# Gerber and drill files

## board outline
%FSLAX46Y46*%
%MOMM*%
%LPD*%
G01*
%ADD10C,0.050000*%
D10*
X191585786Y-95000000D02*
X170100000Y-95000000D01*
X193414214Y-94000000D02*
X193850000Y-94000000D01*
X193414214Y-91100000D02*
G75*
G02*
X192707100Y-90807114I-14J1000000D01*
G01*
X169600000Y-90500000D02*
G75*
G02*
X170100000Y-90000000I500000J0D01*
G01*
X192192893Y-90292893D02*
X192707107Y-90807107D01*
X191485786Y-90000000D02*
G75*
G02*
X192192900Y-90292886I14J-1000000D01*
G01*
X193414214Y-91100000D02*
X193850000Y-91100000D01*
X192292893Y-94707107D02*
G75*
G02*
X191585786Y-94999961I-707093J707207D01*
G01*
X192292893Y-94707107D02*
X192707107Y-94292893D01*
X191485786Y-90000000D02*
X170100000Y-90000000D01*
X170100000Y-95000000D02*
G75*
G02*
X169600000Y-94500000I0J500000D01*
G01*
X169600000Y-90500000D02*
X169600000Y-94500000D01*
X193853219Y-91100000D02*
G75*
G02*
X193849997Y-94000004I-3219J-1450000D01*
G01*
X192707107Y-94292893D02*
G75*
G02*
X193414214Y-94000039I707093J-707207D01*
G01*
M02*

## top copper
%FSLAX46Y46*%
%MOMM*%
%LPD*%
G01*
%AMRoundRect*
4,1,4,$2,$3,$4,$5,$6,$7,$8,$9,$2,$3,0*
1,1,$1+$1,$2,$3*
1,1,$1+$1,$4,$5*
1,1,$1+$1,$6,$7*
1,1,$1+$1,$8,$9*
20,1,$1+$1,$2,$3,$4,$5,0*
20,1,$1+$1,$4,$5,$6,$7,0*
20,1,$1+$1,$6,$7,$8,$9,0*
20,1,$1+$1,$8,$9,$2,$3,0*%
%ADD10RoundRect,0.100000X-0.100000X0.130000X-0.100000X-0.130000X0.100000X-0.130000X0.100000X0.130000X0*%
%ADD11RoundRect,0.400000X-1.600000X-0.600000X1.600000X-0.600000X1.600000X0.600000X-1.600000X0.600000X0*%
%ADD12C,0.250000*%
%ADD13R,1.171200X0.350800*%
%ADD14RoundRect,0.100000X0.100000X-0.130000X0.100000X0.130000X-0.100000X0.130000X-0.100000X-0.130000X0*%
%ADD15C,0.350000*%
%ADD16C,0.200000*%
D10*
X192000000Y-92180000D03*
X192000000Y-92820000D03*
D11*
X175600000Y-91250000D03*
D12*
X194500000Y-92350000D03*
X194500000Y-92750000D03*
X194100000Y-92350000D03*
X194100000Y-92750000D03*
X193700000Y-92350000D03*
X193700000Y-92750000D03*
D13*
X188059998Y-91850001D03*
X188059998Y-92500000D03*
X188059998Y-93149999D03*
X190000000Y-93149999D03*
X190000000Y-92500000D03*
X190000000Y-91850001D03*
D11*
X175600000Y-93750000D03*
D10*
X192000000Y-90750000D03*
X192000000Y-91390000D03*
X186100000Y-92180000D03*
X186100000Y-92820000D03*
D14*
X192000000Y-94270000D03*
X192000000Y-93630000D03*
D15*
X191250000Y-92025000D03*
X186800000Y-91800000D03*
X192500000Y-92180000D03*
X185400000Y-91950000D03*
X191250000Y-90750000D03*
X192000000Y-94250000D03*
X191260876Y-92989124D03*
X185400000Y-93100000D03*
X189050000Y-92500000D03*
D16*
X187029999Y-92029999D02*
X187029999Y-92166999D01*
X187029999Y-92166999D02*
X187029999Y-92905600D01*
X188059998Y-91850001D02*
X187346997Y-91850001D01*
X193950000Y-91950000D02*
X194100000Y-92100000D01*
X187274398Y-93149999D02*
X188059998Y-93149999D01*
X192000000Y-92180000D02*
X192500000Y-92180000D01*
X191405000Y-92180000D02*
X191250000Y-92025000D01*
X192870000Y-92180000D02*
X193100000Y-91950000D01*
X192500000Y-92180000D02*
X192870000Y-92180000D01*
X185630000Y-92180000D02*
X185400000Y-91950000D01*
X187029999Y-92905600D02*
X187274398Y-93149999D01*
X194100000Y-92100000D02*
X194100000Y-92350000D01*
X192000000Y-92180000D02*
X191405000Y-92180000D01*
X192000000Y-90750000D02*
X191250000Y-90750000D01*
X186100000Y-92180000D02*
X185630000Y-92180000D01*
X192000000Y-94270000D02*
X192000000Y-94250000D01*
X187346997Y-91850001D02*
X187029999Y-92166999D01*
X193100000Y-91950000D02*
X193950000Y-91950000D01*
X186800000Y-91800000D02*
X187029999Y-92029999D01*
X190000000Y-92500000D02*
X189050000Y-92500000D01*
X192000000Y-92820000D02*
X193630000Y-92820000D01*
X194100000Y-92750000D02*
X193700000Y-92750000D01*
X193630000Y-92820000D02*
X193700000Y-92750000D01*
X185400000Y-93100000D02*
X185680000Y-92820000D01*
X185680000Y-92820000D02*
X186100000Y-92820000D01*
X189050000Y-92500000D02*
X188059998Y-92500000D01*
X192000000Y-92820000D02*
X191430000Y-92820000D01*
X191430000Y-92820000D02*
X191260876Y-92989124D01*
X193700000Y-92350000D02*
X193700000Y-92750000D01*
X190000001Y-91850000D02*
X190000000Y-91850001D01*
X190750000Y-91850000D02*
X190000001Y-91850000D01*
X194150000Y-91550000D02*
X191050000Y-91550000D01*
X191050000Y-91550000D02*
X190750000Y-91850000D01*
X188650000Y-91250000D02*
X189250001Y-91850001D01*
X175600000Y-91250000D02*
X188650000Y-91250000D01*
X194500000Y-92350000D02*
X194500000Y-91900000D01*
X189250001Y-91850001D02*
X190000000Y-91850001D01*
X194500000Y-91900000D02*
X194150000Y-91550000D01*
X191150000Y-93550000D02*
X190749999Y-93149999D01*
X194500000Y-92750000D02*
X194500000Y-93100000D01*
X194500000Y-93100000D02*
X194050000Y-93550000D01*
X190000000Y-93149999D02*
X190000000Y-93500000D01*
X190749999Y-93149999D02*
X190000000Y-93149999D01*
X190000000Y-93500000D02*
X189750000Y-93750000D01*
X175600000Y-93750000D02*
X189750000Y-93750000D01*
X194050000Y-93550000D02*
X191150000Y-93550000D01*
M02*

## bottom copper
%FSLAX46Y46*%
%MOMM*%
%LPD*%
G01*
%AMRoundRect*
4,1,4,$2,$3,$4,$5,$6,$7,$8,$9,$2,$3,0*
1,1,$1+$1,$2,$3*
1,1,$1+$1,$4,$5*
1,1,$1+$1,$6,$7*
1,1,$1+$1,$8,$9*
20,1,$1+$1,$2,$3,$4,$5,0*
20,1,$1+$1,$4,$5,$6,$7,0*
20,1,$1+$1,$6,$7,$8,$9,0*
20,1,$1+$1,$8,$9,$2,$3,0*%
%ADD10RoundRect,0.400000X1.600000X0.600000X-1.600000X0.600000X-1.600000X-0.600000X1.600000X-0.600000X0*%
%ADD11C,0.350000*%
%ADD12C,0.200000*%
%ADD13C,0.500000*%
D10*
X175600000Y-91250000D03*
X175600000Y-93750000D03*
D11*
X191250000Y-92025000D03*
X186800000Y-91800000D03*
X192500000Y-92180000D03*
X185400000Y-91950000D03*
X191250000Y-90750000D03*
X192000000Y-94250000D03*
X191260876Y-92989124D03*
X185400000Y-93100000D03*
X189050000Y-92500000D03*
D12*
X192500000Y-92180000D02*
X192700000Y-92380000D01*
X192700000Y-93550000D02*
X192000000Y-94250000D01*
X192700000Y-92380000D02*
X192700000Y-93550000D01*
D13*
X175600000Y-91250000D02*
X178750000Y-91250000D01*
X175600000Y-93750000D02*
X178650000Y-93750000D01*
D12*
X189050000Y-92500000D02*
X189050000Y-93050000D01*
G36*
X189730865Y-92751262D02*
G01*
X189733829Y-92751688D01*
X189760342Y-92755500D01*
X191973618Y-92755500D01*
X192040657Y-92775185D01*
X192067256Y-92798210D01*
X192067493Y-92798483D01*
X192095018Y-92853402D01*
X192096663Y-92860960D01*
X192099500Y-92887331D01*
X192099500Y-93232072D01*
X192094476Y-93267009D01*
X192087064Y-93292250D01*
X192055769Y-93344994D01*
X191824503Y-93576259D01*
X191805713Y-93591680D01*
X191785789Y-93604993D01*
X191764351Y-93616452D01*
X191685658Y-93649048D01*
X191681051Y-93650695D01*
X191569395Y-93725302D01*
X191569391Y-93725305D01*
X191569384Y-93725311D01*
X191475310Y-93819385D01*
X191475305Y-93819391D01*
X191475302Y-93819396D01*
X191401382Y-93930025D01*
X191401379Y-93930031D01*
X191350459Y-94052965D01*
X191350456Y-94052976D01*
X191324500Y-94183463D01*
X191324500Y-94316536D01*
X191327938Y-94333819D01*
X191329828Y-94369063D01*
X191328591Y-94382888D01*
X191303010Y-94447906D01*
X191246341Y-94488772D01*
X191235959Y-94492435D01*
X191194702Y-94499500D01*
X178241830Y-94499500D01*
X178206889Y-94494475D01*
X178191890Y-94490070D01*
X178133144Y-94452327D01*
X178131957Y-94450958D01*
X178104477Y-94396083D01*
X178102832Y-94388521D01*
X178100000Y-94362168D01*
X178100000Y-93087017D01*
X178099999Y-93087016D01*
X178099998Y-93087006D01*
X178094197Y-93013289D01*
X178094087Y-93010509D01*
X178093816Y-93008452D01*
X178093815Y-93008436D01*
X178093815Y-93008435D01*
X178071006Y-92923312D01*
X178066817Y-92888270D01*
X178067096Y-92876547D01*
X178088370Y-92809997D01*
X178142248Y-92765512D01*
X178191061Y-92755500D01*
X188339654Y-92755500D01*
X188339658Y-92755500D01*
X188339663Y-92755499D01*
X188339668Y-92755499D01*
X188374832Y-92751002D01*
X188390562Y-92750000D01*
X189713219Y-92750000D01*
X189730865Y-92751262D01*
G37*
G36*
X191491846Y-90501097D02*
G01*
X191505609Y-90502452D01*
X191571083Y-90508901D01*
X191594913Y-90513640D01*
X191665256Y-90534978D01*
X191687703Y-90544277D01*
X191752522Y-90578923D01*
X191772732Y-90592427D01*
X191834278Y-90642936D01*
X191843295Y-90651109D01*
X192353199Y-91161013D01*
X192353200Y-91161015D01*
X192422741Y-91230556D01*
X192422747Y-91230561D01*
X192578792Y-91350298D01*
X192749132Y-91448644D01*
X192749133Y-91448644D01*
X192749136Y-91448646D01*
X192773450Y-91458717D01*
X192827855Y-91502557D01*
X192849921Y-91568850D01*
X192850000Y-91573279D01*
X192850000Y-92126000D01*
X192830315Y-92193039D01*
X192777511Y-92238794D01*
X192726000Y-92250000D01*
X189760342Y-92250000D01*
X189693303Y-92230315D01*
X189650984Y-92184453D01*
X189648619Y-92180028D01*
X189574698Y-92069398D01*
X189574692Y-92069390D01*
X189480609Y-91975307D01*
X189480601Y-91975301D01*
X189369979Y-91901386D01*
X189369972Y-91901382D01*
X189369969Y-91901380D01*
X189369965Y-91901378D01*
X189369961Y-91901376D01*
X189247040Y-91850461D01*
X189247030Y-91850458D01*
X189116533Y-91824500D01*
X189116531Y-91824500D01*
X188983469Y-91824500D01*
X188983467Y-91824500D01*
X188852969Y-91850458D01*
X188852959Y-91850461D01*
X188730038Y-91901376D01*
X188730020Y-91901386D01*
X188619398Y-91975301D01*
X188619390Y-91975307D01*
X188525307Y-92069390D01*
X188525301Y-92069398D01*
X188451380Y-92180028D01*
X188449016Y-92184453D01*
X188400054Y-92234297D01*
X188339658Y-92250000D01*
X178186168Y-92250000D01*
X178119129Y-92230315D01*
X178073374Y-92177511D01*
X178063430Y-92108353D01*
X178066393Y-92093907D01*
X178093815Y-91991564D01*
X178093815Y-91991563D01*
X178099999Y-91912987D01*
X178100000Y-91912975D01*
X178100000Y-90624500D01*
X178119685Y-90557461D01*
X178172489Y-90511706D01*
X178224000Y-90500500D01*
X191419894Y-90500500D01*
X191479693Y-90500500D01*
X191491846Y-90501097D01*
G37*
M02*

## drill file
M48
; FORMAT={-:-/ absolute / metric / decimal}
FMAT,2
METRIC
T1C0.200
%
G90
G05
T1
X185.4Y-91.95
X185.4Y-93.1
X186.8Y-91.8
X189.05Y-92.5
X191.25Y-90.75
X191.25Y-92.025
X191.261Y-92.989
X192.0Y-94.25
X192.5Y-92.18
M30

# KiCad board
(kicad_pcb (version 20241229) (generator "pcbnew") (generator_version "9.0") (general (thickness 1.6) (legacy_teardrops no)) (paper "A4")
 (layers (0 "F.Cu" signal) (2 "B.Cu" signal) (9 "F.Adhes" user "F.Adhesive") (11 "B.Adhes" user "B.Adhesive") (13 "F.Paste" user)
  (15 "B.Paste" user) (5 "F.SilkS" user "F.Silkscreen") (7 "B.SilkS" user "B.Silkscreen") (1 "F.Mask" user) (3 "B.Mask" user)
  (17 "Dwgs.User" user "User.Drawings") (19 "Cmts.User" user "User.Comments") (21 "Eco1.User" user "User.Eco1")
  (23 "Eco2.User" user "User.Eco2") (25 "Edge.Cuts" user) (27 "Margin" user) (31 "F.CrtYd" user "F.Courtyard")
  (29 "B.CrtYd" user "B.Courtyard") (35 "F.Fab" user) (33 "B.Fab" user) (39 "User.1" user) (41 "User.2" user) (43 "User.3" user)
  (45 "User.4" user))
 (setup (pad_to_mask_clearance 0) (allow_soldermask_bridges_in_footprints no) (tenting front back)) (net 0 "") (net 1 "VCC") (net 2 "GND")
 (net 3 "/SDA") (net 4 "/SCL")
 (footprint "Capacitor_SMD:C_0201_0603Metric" (layer "F.Cu") (at 192 92.5 -90)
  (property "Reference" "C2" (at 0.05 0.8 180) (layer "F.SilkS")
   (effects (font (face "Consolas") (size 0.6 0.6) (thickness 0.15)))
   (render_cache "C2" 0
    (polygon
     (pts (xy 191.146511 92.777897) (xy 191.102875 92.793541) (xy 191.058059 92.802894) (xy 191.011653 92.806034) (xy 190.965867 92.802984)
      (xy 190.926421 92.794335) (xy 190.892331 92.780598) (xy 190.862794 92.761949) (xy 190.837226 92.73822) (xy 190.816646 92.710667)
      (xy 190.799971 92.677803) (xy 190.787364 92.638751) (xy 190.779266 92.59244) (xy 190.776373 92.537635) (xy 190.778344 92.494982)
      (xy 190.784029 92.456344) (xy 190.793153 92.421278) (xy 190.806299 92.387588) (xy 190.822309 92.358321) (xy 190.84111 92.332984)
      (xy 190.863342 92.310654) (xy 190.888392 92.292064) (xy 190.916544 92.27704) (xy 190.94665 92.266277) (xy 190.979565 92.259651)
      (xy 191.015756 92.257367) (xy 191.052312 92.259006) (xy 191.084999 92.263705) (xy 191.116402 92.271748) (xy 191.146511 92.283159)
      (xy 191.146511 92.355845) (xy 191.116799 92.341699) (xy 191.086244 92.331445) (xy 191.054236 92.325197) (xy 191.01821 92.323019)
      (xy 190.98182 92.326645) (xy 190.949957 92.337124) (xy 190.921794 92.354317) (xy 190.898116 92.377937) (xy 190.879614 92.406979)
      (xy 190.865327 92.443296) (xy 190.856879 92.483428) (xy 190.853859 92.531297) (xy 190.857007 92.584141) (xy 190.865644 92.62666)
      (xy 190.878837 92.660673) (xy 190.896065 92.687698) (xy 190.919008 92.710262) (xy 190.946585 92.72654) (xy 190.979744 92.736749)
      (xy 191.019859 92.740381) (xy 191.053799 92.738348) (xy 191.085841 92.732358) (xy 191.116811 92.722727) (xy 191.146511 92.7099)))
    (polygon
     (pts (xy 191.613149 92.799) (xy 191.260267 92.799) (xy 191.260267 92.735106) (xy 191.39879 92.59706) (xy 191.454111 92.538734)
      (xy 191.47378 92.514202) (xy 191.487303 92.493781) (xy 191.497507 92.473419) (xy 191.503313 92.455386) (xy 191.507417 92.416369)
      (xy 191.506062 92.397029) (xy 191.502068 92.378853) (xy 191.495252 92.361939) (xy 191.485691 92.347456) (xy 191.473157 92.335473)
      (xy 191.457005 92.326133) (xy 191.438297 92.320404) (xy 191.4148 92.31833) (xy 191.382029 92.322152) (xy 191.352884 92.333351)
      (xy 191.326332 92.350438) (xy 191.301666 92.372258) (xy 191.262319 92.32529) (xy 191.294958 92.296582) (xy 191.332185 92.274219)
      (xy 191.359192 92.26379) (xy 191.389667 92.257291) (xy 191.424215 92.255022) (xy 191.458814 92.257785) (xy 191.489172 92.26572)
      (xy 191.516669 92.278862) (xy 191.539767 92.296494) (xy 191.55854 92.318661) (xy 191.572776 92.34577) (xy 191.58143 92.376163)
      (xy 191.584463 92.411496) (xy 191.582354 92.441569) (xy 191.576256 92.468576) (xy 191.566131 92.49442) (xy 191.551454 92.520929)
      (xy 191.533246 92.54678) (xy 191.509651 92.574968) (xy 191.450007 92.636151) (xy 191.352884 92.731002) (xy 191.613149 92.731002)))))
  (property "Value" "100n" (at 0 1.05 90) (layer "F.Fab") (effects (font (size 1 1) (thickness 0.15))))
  (pad "" smd roundrect (at -0.345 0 270) (size 0.318 0.36) (layers "F.Paste") (roundrect_rratio 0.25))
  (pad "" smd roundrect (at 0.345 0 270) (size 0.318 0.36) (layers "F.Paste") (roundrect_rratio 0.25))
  (pad "1" smd roundrect (at -0.32 0 270) (size 0.46 0.4) (layers "F.Cu" "F.Mask") (roundrect_rratio 0.25) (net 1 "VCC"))
  (pad "2" smd roundrect (at 0.32 0 270) (size 0.46 0.4) (layers "F.Cu" "F.Mask") (roundrect_rratio 0.25) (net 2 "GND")))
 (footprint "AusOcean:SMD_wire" (layer "F.Cu") (at 175.6 91.25)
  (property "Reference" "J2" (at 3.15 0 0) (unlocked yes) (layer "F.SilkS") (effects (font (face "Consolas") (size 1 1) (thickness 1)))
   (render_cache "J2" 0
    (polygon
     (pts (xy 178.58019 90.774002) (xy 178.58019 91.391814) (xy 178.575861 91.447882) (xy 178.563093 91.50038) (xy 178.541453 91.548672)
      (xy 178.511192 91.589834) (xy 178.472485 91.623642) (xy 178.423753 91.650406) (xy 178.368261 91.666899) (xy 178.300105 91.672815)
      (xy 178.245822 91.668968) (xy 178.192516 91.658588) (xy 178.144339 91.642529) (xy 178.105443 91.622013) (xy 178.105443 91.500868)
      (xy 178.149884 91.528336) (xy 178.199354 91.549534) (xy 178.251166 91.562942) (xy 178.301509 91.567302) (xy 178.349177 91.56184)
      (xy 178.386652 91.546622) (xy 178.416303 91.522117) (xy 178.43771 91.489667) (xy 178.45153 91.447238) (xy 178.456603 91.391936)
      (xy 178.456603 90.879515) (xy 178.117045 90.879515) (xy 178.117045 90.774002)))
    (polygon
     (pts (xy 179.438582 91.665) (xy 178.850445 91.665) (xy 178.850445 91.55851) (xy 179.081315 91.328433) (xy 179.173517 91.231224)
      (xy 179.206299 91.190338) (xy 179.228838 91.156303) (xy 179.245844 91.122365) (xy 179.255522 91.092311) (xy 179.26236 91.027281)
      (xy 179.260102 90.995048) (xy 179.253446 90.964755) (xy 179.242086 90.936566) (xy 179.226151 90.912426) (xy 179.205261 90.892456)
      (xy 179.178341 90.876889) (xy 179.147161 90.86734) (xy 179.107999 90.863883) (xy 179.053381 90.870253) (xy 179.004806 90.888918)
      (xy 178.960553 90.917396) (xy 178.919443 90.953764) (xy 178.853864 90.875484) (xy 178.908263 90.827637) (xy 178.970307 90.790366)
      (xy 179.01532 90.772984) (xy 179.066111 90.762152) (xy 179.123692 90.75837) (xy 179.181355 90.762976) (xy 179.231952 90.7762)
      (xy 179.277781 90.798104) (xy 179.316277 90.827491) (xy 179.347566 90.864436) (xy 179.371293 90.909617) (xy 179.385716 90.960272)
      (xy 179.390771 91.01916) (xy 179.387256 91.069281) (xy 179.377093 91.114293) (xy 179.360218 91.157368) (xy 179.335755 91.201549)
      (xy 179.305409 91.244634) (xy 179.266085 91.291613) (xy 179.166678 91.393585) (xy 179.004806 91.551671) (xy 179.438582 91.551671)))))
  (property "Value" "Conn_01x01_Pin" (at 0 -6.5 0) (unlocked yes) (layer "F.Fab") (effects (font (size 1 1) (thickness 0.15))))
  (pad "1" smd roundrect (at 0 0) (size 4 2) (layers "F.Cu" "F.Mask" "F.Paste") (roundrect_rratio 0.2) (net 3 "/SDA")
   (thermal_bridge_angle 45)))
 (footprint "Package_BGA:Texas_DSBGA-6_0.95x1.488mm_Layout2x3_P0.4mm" (layer "F.Cu") (at 194.1 92.55 -90)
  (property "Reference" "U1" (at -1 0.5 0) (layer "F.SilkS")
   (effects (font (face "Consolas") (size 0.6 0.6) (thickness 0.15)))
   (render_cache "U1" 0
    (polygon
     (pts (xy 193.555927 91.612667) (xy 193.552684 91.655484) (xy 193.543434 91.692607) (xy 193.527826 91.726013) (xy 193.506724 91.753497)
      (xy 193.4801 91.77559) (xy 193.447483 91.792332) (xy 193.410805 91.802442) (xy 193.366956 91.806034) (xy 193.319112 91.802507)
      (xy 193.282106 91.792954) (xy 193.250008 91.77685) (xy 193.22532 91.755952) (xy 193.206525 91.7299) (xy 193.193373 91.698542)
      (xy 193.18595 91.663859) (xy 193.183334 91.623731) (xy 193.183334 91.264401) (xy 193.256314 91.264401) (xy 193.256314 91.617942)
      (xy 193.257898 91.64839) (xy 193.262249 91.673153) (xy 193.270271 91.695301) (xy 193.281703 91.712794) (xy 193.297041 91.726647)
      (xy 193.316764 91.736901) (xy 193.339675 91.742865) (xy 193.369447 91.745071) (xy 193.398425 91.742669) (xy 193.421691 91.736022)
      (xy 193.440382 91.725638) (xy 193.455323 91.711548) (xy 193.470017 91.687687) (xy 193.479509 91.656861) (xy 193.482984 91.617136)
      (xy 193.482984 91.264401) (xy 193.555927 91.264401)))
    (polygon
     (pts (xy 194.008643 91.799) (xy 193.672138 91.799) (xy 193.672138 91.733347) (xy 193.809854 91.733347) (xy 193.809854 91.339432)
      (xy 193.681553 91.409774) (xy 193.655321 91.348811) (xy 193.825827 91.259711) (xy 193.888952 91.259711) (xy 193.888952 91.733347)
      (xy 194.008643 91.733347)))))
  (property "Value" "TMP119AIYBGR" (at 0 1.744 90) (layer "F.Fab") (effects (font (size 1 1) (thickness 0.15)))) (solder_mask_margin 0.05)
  (pad "A1" smd circle (at -0.2 -0.4 270) (size 0.25 0.25) (layers "F.Cu" "F.Mask" "F.Paste") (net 3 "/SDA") (clearance 0.05))
  (pad "A2" smd circle (at 0.2 -0.4 270) (size 0.25 0.25) (layers "F.Cu" "F.Mask" "F.Paste") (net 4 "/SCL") (clearance 0.05))
  (pad "B1" smd circle (at -0.2 0 270) (size 0.25 0.25) (layers "F.Cu" "F.Mask" "F.Paste") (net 1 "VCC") (clearance 0.05))
  (pad "B2" smd circle (at 0.2 0 270) (size 0.25 0.25) (layers "F.Cu" "F.Mask" "F.Paste") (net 2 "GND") (clearance 0.05))
  (pad "C1" smd circle (at -0.2 0.4 270) (size 0.25 0.25) (layers "F.Cu" "F.Mask" "F.Paste") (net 2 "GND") (clearance 0.05))
  (pad "C2" smd circle (at 0.2 0.4 270) (size 0.25 0.25) (layers "F.Cu" "F.Mask" "F.Paste") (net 2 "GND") (clearance 0.05)))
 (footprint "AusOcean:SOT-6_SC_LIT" (layer "F.Cu") (at 189.029999 92.5)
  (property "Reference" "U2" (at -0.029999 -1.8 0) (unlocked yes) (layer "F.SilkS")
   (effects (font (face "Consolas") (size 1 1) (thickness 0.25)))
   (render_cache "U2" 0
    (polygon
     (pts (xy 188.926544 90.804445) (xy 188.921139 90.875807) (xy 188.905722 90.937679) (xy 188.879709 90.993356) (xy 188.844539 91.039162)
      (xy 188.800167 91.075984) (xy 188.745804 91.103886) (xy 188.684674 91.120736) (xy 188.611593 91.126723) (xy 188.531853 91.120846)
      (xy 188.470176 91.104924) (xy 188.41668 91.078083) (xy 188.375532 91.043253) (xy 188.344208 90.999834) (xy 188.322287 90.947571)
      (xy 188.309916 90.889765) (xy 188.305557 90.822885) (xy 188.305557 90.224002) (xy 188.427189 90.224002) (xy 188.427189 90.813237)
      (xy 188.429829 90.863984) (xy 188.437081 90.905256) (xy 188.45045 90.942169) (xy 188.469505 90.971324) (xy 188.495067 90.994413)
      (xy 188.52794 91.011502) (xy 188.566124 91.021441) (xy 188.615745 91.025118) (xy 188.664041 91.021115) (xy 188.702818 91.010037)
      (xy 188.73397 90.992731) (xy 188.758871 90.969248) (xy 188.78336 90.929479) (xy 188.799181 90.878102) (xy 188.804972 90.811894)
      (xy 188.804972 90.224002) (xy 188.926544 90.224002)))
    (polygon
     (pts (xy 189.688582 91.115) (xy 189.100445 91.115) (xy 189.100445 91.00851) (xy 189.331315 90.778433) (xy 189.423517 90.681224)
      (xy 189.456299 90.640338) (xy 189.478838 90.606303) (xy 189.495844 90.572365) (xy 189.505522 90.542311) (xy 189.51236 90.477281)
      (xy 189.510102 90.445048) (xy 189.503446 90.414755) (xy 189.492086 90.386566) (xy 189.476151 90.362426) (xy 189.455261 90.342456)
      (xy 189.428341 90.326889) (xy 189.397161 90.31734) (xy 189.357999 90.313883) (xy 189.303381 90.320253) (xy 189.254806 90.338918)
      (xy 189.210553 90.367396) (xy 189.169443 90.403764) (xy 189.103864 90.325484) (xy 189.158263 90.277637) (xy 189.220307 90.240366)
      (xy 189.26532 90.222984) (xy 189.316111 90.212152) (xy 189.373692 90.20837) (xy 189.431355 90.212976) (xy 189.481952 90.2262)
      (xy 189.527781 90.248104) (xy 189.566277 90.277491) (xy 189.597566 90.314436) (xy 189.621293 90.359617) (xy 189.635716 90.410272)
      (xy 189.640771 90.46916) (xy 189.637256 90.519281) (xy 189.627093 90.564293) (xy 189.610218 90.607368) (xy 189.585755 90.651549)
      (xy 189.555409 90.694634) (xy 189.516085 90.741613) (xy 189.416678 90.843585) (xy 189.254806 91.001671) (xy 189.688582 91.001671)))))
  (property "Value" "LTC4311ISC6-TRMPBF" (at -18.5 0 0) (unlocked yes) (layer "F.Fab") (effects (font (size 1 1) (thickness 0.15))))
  (pad "1" smd rect (at -0.970001 -0.649999) (size 1.1712 0.3508) (layers "F.Cu" "F.Mask" "F.Paste") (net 1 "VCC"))
  (pad "2" smd rect (at -0.970001 0) (size 1.1712 0.3508) (layers "F.Cu" "F.Mask" "F.Paste") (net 2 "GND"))
  (pad "3" smd rect (at -0.970001 0.649999) (size 1.1712 0.3508) (layers "F.Cu" "F.Mask" "F.Paste") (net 1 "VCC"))
  (pad "4" smd rect (at 0.970001 0.649999) (size 1.1712 0.3508) (layers "F.Cu" "F.Mask" "F.Paste") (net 4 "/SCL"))
  (pad "5" smd rect (at 0.970001 0) (size 1.1712 0.3508) (layers "F.Cu" "F.Mask" "F.Paste") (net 2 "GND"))
  (pad "6" smd rect (at 0.970001 -0.649999) (size 1.1712 0.3508) (layers "F.Cu" "F.Mask" "F.Paste") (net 3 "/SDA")))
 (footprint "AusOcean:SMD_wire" (layer "F.Cu") (at 175.6 93.75)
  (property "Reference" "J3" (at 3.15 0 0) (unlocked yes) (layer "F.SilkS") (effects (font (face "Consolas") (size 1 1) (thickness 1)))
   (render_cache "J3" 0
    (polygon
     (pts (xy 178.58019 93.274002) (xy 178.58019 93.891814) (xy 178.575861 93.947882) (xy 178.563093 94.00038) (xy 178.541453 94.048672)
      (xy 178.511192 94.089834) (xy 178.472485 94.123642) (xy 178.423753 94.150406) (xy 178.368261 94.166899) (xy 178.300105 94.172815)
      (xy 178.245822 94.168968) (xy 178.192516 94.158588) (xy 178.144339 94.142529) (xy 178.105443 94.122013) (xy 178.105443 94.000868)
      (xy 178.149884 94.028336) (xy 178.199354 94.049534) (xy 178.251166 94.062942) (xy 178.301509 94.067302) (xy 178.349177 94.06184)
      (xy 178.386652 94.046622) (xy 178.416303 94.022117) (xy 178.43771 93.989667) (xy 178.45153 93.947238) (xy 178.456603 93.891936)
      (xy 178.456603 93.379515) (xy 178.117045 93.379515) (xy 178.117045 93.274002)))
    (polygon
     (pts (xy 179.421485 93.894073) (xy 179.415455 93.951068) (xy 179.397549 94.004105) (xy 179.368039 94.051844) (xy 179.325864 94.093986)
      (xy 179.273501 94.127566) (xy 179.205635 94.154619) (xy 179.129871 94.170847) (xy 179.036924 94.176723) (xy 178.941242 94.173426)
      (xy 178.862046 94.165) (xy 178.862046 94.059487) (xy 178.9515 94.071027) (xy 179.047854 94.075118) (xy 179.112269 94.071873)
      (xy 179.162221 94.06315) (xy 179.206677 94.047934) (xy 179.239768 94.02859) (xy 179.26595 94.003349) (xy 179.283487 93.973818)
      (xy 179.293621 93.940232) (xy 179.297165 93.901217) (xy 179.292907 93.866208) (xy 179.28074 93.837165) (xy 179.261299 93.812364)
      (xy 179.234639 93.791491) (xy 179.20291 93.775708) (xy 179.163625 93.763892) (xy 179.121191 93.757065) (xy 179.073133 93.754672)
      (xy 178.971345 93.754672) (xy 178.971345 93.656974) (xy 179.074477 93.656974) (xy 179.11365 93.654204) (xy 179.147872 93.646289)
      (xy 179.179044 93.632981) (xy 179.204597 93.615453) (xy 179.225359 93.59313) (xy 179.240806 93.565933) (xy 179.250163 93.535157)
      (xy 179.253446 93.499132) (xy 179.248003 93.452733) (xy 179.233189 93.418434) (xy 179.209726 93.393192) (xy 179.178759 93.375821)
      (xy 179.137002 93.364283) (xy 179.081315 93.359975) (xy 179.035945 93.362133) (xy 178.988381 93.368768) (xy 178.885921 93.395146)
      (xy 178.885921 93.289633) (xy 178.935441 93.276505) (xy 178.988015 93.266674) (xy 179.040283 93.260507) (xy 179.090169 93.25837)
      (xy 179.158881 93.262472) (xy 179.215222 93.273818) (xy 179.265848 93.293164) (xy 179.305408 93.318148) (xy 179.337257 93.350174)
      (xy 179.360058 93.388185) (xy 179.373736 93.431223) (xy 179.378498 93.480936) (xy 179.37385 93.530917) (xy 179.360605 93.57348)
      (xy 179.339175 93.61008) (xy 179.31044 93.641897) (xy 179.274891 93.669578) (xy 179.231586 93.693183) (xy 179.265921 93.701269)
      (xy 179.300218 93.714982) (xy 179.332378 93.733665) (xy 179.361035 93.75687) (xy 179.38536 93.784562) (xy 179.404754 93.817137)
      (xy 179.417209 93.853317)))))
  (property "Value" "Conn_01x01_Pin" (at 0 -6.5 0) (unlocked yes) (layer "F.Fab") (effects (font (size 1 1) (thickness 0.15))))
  (pad "1" smd roundrect (at 0 0) (size 4 2) (layers "F.Cu" "F.Mask" "F.Paste") (roundrect_rratio 0.2) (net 4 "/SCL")
   (thermal_bridge_angle 45)))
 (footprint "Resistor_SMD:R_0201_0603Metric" (layer "F.Cu") (at 192 91.07 -90)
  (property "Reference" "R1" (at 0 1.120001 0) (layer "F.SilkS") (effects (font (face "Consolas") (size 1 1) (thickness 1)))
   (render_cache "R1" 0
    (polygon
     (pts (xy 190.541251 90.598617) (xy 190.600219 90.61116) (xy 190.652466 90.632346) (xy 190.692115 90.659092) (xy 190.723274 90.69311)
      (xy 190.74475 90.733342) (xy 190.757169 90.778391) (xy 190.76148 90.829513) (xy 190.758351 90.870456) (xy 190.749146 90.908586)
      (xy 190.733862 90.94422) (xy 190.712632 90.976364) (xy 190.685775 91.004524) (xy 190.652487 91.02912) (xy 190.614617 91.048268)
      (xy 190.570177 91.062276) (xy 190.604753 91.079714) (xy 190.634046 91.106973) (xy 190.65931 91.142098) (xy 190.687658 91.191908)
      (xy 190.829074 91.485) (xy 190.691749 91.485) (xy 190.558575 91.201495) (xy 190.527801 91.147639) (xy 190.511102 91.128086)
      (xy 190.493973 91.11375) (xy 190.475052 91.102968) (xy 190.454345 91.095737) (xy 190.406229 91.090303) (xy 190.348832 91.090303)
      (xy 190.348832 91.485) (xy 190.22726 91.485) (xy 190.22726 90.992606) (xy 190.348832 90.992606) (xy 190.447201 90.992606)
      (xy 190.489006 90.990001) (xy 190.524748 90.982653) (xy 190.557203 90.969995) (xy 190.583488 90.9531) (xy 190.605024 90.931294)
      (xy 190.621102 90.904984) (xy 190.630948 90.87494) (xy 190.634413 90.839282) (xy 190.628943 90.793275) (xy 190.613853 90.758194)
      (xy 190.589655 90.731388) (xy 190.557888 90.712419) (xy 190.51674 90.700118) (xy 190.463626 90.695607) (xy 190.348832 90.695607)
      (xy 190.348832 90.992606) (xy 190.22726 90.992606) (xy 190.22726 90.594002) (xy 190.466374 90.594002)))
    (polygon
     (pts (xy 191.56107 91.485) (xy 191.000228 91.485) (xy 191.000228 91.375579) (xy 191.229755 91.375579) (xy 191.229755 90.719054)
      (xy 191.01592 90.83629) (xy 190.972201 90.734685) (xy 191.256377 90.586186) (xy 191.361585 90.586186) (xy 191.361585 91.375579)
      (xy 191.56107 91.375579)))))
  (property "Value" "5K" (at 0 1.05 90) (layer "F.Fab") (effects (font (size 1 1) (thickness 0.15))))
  (pad "" smd roundrect (at -0.345 0 270) (size 0.318 0.36) (layers "F.Paste") (roundrect_rratio 0.25))
  (pad "" smd roundrect (at 0.345 0 270) (size 0.318 0.36) (layers "F.Paste") (roundrect_rratio 0.25))
  (pad "1" smd roundrect (at -0.32 0 270) (size 0.46 0.4) (layers "F.Cu" "F.Mask") (roundrect_rratio 0.25) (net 1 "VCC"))
  (pad "2" smd roundrect (at 0.32 0 270) (size 0.46 0.4) (layers "F.Cu" "F.Mask") (roundrect_rratio 0.25) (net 3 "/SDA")))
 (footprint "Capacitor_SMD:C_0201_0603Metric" (layer "F.Cu") (at 186.1 92.5 -90)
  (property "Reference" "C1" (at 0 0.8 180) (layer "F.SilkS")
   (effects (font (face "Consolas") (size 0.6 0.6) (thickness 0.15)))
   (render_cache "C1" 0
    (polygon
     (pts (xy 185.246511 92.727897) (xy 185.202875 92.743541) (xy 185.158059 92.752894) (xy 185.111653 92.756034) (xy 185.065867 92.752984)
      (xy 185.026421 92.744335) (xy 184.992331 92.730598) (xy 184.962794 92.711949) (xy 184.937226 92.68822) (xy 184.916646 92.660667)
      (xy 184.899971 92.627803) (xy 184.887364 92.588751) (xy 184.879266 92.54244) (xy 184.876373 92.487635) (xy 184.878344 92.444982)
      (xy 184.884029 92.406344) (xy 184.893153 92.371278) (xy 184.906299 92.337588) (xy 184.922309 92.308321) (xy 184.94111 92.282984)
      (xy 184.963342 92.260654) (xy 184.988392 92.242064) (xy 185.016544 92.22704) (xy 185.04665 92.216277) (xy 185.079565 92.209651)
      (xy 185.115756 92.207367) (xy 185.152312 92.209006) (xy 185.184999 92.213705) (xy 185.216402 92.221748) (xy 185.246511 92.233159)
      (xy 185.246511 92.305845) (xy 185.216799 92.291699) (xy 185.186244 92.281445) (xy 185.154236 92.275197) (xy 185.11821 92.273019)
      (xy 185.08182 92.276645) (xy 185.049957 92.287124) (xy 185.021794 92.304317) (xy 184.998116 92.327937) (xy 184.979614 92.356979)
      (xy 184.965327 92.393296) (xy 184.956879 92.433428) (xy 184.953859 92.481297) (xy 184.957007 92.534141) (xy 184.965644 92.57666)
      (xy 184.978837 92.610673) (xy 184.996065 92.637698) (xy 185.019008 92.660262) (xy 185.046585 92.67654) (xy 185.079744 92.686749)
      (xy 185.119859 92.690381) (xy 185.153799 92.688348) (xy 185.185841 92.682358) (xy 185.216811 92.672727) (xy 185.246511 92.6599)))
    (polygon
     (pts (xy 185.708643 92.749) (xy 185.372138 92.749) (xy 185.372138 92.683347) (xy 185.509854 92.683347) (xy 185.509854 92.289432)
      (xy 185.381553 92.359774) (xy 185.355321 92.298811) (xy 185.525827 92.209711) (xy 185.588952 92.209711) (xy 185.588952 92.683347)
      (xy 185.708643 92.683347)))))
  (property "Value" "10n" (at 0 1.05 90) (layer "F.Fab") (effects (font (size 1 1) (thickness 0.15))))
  (pad "" smd roundrect (at -0.345 0 270) (size 0.318 0.36) (layers "F.Paste") (roundrect_rratio 0.25))
  (pad "" smd roundrect (at 0.345 0 270) (size 0.318 0.36) (layers "F.Paste") (roundrect_rratio 0.25))
  (pad "1" smd roundrect (at -0.32 0 270) (size 0.46 0.4) (layers "F.Cu" "F.Mask") (roundrect_rratio 0.25) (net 1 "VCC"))
  (pad "2" smd roundrect (at 0.32 0 270) (size 0.46 0.4) (layers "F.Cu" "F.Mask") (roundrect_rratio 0.25) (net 2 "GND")))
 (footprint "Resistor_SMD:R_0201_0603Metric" (layer "F.Cu") (at 192 93.95 90)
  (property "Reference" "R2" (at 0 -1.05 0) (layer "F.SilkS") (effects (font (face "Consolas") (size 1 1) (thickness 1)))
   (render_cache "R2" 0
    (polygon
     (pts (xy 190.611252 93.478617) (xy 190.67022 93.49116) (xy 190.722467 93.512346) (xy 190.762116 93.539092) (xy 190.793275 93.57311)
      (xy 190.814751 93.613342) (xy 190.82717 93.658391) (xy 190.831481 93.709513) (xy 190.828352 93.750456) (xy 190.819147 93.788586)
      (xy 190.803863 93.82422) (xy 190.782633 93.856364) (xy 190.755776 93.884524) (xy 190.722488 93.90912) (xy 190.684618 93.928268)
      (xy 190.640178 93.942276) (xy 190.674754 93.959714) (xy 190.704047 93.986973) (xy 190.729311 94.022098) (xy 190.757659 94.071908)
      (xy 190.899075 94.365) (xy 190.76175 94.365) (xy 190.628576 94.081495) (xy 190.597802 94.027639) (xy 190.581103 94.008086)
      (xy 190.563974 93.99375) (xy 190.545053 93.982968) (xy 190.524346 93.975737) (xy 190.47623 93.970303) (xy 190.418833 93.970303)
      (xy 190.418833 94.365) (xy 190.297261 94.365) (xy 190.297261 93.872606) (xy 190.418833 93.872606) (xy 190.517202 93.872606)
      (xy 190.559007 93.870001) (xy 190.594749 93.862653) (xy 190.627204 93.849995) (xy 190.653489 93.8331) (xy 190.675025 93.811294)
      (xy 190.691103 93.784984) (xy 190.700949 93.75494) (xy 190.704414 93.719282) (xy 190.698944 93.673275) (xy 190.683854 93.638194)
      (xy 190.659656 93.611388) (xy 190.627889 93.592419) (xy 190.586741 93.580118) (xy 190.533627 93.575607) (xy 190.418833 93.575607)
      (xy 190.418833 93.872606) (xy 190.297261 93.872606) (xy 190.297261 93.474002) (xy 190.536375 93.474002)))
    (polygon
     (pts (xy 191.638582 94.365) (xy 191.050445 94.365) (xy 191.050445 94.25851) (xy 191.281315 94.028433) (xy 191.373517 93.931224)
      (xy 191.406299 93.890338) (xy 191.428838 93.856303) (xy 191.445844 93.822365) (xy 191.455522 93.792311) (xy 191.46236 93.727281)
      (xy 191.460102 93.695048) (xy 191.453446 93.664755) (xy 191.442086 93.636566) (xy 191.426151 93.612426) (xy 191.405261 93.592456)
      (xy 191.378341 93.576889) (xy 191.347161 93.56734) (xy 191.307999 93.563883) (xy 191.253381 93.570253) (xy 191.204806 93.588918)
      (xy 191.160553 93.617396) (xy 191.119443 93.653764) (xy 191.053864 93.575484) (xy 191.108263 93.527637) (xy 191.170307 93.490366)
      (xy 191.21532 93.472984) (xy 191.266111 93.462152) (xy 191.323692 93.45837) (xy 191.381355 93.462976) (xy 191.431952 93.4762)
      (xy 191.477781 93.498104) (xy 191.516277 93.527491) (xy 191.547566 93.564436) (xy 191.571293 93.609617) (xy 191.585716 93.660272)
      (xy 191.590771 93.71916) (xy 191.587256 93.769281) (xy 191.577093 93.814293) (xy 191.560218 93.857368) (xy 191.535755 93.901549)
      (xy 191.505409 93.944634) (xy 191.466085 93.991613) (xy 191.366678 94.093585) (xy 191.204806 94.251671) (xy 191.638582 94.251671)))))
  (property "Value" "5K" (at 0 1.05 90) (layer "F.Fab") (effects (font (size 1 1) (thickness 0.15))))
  (pad "" smd roundrect (at -0.345 0 90) (size 0.318 0.36) (layers "F.Paste") (roundrect_rratio 0.25))
  (pad "" smd roundrect (at 0.345 0 90) (size 0.318 0.36) (layers "F.Paste") (roundrect_rratio 0.25))
  (pad "1" smd roundrect (at -0.32 0 90) (size 0.46 0.4) (layers "F.Cu" "F.Mask") (roundrect_rratio 0.25) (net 1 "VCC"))
  (pad "2" smd roundrect (at 0.32 0 90) (size 0.46 0.4) (layers "F.Cu" "F.Mask") (roundrect_rratio 0.25) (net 4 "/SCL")))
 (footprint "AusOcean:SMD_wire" (layer "B.Cu") (at 175.6 91.25 180)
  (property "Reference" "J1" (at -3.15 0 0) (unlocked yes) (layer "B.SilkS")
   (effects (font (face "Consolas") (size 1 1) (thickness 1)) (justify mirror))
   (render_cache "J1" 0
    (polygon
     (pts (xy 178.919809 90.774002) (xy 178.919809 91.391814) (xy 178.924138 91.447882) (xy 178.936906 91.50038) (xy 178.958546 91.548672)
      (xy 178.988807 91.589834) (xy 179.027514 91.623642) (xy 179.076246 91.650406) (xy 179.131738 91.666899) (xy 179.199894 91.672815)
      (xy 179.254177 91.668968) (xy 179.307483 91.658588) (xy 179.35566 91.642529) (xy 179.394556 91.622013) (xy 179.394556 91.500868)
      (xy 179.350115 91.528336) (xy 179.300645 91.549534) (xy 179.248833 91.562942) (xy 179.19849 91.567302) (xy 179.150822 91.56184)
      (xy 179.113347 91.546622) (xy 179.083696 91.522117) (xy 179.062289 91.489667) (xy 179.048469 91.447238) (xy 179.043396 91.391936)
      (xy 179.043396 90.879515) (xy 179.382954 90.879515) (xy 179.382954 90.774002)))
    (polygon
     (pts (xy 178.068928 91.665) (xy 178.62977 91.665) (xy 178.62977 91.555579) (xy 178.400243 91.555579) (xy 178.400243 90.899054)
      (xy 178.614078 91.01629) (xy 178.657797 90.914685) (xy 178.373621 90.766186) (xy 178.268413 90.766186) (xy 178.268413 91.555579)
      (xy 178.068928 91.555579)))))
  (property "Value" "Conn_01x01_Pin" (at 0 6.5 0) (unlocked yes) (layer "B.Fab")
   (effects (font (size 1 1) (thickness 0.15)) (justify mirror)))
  (pad "1" smd roundrect (at 0 0 180) (size 4 2) (layers "B.Cu" "B.Mask" "B.Paste") (roundrect_rratio 0.2) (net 1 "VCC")
   (thermal_bridge_angle 45)))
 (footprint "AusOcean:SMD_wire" (layer "B.Cu") (at 175.6 93.75 180)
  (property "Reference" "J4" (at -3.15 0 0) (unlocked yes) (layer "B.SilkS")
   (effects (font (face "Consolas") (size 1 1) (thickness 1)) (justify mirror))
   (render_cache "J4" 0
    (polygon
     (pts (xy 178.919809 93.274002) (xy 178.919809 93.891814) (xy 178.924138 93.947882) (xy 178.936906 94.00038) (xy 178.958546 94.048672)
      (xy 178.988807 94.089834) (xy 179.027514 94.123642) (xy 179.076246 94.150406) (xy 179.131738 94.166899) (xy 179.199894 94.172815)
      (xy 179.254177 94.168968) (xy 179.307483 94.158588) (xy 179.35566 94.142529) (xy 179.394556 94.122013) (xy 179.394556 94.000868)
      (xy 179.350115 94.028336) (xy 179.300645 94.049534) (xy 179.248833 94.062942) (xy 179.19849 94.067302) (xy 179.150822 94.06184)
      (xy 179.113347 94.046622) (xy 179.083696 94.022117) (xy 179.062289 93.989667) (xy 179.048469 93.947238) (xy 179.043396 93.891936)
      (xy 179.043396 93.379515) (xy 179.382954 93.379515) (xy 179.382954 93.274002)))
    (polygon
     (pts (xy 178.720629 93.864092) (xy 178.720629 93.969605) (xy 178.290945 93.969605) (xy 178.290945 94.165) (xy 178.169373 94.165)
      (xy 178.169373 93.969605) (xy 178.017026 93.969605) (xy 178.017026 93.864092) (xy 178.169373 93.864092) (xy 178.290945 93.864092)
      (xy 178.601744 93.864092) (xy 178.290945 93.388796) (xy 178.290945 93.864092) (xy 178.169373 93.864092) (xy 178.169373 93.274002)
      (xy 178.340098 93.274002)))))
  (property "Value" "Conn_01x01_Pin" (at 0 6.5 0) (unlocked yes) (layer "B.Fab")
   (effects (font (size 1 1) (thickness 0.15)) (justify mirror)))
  (pad "1" smd roundrect (at 0 0 180) (size 4 2) (layers "B.Cu" "B.Mask" "B.Paste") (roundrect_rratio 0.2) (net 2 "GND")
   (thermal_bridge_angle 45)))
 (gr_line (start 191.585786 95) (end 170.1 95) (stroke (width 0.05) (type default)) (layer "Edge.Cuts"))
 (gr_line (start 193.414214 94) (end 193.85 94) (stroke (width 0.05) (type default)) (layer "Edge.Cuts"))
 (gr_arc (start 193.414214 91.1) (mid 193.031531 91.02388) (end 192.707107 90.807107) (stroke (width 0.05) (type default))
  (layer "Edge.Cuts"))
 (gr_arc (start 169.6 90.5) (mid 169.746447 90.146447) (end 170.1 90) (stroke (width 0.05) (type default)) (layer "Edge.Cuts"))
 (gr_line (start 192.192893 90.292893) (end 192.707107 90.807107) (stroke (width 0.05) (type default)) (layer "Edge.Cuts"))
 (gr_arc (start 191.485786 90) (mid 191.868469 90.07612) (end 192.192893 90.292893) (stroke (width 0.05) (type default)) (layer "Edge.Cuts"))
 (gr_line (start 193.414214 91.1) (end 193.85 91.1) (stroke (width 0.05) (type default)) (layer "Edge.Cuts"))
 (gr_arc (start 192.292893 94.707107) (mid 191.968469 94.923875) (end 191.585786 95) (stroke (width 0.05) (type default))
  (layer "Edge.Cuts"))
 (gr_line (start 192.292893 94.707107) (end 192.707107 94.292893) (stroke (width 0.05) (type default)) (layer "Edge.Cuts"))
 (gr_line (start 191.485786 90) (end 170.1 90) (stroke (width 0.05) (type default)) (layer "Edge.Cuts"))
 (gr_arc (start 170.1 95) (mid 169.746447 94.853553) (end 169.6 94.5) (stroke (width 0.05) (type default)) (layer "Edge.Cuts"))
 (gr_line (start 169.6 90.5) (end 169.6 94.5) (stroke (width 0.05) (type default)) (layer "Edge.Cuts"))
 (gr_arc (start 193.853219 91.1) (mid 195.3 92.551611) (end 193.849997 94.000004) (stroke (width 0.05) (type default)) (layer "Edge.Cuts"))
 (gr_arc (start 192.707107 94.292893) (mid 193.031531 94.076125) (end 193.414214 94) (stroke (width 0.05) (type default))
  (layer "Edge.Cuts"))
 (segment (start 187.029999 92.029999) (end 187.029999 92.166999) (width 0.2) (layer "F.Cu") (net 1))
 (segment (start 187.029999 92.166999) (end 187.029999 92.9056) (width 0.2) (layer "F.Cu") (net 1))
 (segment (start 188.059998 91.850001) (end 187.346997 91.850001) (width 0.2) (layer "F.Cu") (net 1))
 (segment (start 193.95 91.95) (end 194.1 92.1) (width 0.2) (layer "F.Cu") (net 1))
 (segment (start 187.274398 93.149999) (end 188.059998 93.149999) (width 0.2) (layer "F.Cu") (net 1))
 (segment (start 192 92.18) (end 192.5 92.18) (width 0.2) (layer "F.Cu") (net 1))
 (segment (start 191.405 92.18) (end 191.25 92.025) (width 0.2) (layer "F.Cu") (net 1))
 (segment (start 192.87 92.18) (end 193.1 91.95) (width 0.2) (layer "F.Cu") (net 1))
 (segment (start 192.5 92.18) (end 192.87 92.18) (width 0.2) (layer "F.Cu") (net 1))
 (segment (start 185.63 92.18) (end 185.4 91.95) (width 0.2) (layer "F.Cu") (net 1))
 (segment (start 187.029999 92.9056) (end 187.274398 93.149999) (width 0.2) (layer "F.Cu") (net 1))
 (segment (start 194.1 92.1) (end 194.1 92.35) (width 0.2) (layer "F.Cu") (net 1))
 (segment (start 192 92.18) (end 191.405 92.18) (width 0.2) (layer "F.Cu") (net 1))
 (segment (start 192 90.75) (end 191.25 90.75) (width 0.2) (layer "F.Cu") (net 1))
 (segment (start 186.1 92.18) (end 185.63 92.18) (width 0.2) (layer "F.Cu") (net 1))
 (segment (start 192 94.27) (end 192 94.25) (width 0.2) (layer "F.Cu") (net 1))
 (segment (start 187.346997 91.850001) (end 187.029999 92.166999) (width 0.2) (layer "F.Cu") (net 1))
 (segment (start 193.1 91.95) (end 193.95 91.95) (width 0.2) (layer "F.Cu") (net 1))
 (segment (start 186.8 91.8) (end 187.029999 92.029999) (width 0.2) (layer "F.Cu") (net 1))
 (via (at 191.25 92.025) (size 0.35) (drill 0.2) (layers "F.Cu" "B.Cu") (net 1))
 (via (at 186.8 91.8) (size 0.35) (drill 0.2) (layers "F.Cu" "B.Cu") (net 1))
 (via (at 192.5 92.18) (size 0.35) (drill 0.2) (layers "F.Cu" "B.Cu") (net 1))
 (via (at 185.4 91.95) (size 0.35) (drill 0.2) (layers "F.Cu" "B.Cu") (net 1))
 (via (at 191.25 90.75) (size 0.35) (drill 0.2) (layers "F.Cu" "B.Cu") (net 1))
 (via (at 192 94.25) (size 0.35) (drill 0.2) (layers "F.Cu" "B.Cu") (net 1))
 (segment (start 192.5 92.18) (end 192.7 92.38) (width 0.2) (layer "B.Cu") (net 1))
 (segment (start 192.7 93.55) (end 192 94.25) (width 0.2) (layer "B.Cu") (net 1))
 (segment (start 192.7 92.38) (end 192.7 93.55) (width 0.2) (layer "B.Cu") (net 1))
 (segment (start 175.6 91.25) (end 178.75 91.25) (width 0.5) (layer "B.Cu") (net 1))
 (segment (start 190 92.5) (end 189.05 92.5) (width 0.2) (layer "F.Cu") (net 2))
 (segment (start 192 92.82) (end 193.63 92.82) (width 0.2) (layer "F.Cu") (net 2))
 (segment (start 194.1 92.75) (end 193.7 92.75) (width 0.2) (layer "F.Cu") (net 2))
 (segment (start 193.63 92.82) (end 193.7 92.75) (width 0.2) (layer "F.Cu") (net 2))
 (segment (start 185.4 93.1) (end 185.68 92.82) (width 0.2) (layer "F.Cu") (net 2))
 (segment (start 185.68 92.82) (end 186.1 92.82) (width 0.2) (layer "F.Cu") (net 2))
 (segment (start 189.05 92.5) (end 188.059998 92.5) (width 0.2) (layer "F.Cu") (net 2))
 (segment (start 192 92.82) (end 191.43 92.82) (width 0.2) (layer "F.Cu") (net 2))
 (segment (start 191.43 92.82) (end 191.260876 92.989124) (width 0.2) (layer "F.Cu") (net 2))
 (segment (start 193.7 92.35) (end 193.7 92.75) (width 0.2) (layer "F.Cu") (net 2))
 (via (at 191.260876 92.989124) (size 0.35) (drill 0.2) (layers "F.Cu" "B.Cu") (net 2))
 (via (at 185.4 93.1) (size 0.35) (drill 0.2) (layers "F.Cu" "B.Cu") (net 2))
 (via (at 189.05 92.5) (size 0.35) (drill 0.2) (layers "F.Cu" "B.Cu") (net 2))
 (segment (start 175.6 93.75) (end 178.65 93.75) (width 0.5) (layer "B.Cu") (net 2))
 (segment (start 189.05 92.5) (end 189.05 93.05) (width 0.2) (layer "B.Cu") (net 2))
 (segment (start 190.000001 91.85) (end 190 91.850001) (width 0.2) (layer "F.Cu") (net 3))
 (segment (start 190.75 91.85) (end 190.000001 91.85) (width 0.2) (layer "F.Cu") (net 3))
 (segment (start 194.15 91.55) (end 191.05 91.55) (width 0.2) (layer "F.Cu") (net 3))
 (segment (start 191.05 91.55) (end 190.75 91.85) (width 0.2) (layer "F.Cu") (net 3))
 (segment (start 188.65 91.25) (end 189.250001 91.850001) (width 0.2) (layer "F.Cu") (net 3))
 (segment (start 175.6 91.25) (end 188.65 91.25) (width 0.2) (layer "F.Cu") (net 3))
 (segment (start 194.5 92.35) (end 194.5 91.9) (width 0.2) (layer "F.Cu") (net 3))
 (segment (start 189.250001 91.850001) (end 190 91.850001) (width 0.2) (layer "F.Cu") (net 3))
 (segment (start 194.5 91.9) (end 194.15 91.55) (width 0.2) (layer "F.Cu") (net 3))
 (segment (start 191.15 93.55) (end 190.749999 93.149999) (width 0.2) (layer "F.Cu") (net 4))
 (segment (start 194.5 92.75) (end 194.5 93.1) (width 0.2) (layer "F.Cu") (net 4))
 (segment (start 194.5 93.1) (end 194.05 93.55) (width 0.2) (layer "F.Cu") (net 4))
 (segment (start 190 93.149999) (end 190 93.5) (width 0.2) (layer "F.Cu") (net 4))
 (segment (start 190.749999 93.149999) (end 190 93.149999) (width 0.2) (layer "F.Cu") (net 4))
 (segment (start 190 93.5) (end 189.75 93.75) (width 0.2) (layer "F.Cu") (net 4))
 (segment (start 175.6 93.75) (end 189.75 93.75) (width 0.2) (layer "F.Cu") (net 4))
 (segment (start 194.05 93.55) (end 191.15 93.55) (width 0.2) (layer "F.Cu") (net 4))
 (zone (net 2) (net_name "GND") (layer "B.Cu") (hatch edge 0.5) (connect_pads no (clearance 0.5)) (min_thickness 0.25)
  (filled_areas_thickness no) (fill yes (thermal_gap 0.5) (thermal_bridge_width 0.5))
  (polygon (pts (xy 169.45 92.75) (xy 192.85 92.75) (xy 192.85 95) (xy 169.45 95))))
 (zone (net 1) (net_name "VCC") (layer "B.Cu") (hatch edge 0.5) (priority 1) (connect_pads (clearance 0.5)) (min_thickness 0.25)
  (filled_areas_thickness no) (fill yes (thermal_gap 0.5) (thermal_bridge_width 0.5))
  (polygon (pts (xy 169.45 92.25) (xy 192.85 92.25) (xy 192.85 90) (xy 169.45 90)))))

